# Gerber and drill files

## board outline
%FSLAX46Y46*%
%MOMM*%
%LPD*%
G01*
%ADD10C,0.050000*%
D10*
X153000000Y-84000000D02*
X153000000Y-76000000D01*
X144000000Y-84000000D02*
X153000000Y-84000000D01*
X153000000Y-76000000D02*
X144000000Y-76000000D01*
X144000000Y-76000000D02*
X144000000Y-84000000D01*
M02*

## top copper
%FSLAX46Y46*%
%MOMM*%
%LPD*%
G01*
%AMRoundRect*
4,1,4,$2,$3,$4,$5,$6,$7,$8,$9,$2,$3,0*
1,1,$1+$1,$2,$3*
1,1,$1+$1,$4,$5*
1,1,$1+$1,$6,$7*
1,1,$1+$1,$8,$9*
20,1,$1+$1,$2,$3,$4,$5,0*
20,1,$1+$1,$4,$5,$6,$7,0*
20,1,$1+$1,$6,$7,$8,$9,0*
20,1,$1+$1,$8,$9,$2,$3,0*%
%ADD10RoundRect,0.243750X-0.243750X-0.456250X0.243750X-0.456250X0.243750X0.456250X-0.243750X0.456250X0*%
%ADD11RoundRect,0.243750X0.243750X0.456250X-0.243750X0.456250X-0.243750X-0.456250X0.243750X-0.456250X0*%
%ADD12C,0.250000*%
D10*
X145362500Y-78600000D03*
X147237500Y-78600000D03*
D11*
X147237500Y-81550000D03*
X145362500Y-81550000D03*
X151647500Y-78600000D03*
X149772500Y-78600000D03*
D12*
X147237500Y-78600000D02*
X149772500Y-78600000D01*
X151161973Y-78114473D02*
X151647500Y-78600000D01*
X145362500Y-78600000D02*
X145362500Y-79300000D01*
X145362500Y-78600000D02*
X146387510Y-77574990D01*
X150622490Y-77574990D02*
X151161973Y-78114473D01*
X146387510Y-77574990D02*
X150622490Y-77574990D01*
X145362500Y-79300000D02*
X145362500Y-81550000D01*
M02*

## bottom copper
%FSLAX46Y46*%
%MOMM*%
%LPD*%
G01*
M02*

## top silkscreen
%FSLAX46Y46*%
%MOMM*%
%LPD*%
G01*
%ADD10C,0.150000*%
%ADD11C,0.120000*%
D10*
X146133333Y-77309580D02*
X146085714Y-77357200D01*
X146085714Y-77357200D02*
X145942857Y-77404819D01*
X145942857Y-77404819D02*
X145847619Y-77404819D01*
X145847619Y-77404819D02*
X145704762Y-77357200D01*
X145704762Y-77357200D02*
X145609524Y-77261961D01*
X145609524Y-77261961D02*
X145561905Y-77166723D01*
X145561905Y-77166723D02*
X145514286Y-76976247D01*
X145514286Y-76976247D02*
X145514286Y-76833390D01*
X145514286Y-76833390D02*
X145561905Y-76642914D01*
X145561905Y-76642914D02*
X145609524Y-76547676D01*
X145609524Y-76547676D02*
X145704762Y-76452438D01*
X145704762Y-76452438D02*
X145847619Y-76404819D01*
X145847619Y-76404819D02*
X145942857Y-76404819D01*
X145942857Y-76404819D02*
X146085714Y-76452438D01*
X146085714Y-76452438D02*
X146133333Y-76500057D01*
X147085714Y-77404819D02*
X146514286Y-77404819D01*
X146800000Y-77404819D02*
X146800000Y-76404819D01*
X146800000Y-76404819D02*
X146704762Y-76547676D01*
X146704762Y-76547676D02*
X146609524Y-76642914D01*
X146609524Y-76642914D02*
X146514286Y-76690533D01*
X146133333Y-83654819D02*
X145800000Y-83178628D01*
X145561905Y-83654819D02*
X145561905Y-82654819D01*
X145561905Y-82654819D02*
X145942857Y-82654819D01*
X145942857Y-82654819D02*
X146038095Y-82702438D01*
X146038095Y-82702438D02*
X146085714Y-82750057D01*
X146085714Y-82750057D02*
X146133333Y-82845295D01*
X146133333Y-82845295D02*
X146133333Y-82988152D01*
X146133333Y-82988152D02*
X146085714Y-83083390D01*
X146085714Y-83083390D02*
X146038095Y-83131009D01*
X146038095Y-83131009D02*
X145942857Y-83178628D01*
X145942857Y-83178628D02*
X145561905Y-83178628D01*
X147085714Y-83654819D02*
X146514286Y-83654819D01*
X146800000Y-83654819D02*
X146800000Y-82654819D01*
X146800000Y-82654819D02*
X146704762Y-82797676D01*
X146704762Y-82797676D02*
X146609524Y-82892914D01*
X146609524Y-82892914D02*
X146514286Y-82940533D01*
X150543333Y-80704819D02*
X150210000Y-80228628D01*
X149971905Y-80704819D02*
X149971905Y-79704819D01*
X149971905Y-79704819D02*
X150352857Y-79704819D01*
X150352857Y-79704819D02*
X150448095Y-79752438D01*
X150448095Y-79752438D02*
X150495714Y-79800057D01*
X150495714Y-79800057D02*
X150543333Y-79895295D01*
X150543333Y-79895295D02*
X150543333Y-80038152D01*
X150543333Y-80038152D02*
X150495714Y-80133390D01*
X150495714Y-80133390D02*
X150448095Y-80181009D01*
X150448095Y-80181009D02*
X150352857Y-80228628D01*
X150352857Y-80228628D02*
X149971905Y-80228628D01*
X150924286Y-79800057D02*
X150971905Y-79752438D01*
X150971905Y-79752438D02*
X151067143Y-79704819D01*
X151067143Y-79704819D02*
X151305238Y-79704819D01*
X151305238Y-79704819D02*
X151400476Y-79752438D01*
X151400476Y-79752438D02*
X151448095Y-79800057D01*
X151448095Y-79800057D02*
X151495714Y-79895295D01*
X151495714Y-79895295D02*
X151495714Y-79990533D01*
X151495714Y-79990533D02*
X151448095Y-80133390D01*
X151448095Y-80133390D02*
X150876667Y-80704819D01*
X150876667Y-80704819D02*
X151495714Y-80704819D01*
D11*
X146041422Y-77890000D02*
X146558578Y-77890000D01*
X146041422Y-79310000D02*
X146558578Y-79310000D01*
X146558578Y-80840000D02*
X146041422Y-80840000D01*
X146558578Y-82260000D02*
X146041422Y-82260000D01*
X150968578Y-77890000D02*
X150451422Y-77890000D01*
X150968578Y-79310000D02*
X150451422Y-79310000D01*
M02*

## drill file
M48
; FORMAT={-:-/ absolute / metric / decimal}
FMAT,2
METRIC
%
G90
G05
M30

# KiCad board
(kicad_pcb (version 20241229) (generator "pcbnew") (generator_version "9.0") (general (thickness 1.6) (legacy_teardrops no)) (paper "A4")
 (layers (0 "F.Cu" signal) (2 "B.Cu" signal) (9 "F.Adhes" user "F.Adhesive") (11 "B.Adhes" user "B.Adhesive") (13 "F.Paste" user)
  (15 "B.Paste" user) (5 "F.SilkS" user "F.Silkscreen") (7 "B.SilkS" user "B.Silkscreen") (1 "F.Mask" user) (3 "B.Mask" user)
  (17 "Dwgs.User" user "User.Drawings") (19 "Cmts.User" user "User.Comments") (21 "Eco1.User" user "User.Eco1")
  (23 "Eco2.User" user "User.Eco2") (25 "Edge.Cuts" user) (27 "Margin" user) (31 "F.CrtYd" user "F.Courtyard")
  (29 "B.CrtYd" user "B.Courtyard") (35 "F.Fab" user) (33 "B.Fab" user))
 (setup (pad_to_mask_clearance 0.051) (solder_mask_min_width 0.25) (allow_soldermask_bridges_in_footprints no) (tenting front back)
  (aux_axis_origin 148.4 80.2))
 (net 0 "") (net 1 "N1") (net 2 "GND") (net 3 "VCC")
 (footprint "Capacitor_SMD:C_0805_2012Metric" (layer "F.Cu") (at 146.3 78.6)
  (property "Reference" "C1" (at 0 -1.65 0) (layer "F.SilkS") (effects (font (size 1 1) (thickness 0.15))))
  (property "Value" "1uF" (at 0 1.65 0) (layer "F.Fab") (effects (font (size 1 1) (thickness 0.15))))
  (fp_line (start -0.258578 -0.71) (end 0.258578 -0.71) (stroke (width 0.12) (type solid)) (layer "F.SilkS"))
  (fp_line (start -0.258578 0.71) (end 0.258578 0.71) (stroke (width 0.12) (type solid)) (layer "F.SilkS"))
  (pad "1" smd roundrect (at -0.9375 0) (size 0.975 1.4) (layers "F.Cu" "F.Mask" "F.Paste") (roundrect_rratio 0.25) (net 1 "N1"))
  (pad "2" smd roundrect (at 0.9375 0) (size 0.975 1.4) (layers "F.Cu" "F.Mask" "F.Paste") (roundrect_rratio 0.25) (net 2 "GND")))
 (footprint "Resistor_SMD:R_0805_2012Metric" (layer "F.Cu") (at 146.3 81.55 180)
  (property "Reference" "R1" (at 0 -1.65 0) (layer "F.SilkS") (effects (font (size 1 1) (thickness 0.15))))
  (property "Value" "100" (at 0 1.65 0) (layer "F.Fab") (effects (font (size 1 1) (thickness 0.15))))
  (fp_line (start -0.258578 0.71) (end 0.258578 0.71) (stroke (width 0.12) (type solid)) (layer "F.SilkS"))
  (fp_line (start -0.258578 -0.71) (end 0.258578 -0.71) (stroke (width 0.12) (type solid)) (layer "F.SilkS"))
  (pad "1" smd roundrect (at -0.9375 0 180) (size 0.975 1.4) (layers "F.Cu" "F.Mask" "F.Paste") (roundrect_rratio 0.25) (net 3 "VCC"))
  (pad "2" smd roundrect (at 0.9375 0 180) (size 0.975 1.4) (layers "F.Cu" "F.Mask" "F.Paste") (roundrect_rratio 0.25) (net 1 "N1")))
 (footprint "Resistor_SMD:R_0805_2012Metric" (layer "F.Cu") (at 150.71 78.6 180)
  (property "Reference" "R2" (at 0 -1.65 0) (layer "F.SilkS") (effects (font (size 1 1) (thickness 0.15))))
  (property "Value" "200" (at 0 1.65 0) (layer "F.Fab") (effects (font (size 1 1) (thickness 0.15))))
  (fp_line (start -0.258578 0.71) (end 0.258578 0.71) (stroke (width 0.12) (type solid)) (layer "F.SilkS"))
  (fp_line (start -0.258578 -0.71) (end 0.258578 -0.71) (stroke (width 0.12) (type solid)) (layer "F.SilkS"))
  (pad "1" smd roundrect (at -0.9375 0 180) (size 0.975 1.4) (layers "F.Cu" "F.Mask" "F.Paste") (roundrect_rratio 0.25) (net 1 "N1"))
  (pad "2" smd roundrect (at 0.9375 0 180) (size 0.975 1.4) (layers "F.Cu" "F.Mask" "F.Paste") (roundrect_rratio 0.25) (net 2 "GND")))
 (gr_line (start 153 84) (end 153 76) (stroke (width 0.05) (type solid)) (layer "Edge.Cuts"))
 (gr_line (start 144 84) (end 153 84) (stroke (width 0.05) (type solid)) (layer "Edge.Cuts"))
 (gr_line (start 153 76) (end 144 76) (stroke (width 0.05) (type solid)) (layer "Edge.Cuts"))
 (gr_line (start 144 76) (end 144 84) (stroke (width 0.05) (type solid)) (layer "Edge.Cuts"))
 (segment (start 147.2375 78.6) (end 149.7725 78.6) (width 0.25) (layer "F.Cu") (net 2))
 (segment (start 151.161973 78.114473) (end 151.6475 78.6) (width 0.25) (layer "F.Cu") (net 1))
 (segment (start 145.3625 78.6) (end 145.3625 79.3) (width 0.25) (layer "F.Cu") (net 1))
 (segment (start 145.3625 78.6) (end 146.38751 77.57499) (width 0.25) (layer "F.Cu") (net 1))
 (segment (start 150.62249 77.57499) (end 151.161973 78.114473) (width 0.25) (layer "F.Cu") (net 1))
 (segment (start 146.38751 77.57499) (end 150.62249 77.57499) (width 0.25) (layer "F.Cu") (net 1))
 (segment (start 145.3625 79.3) (end 145.3625 81.55) (width 0.25) (layer "F.Cu") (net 1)))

